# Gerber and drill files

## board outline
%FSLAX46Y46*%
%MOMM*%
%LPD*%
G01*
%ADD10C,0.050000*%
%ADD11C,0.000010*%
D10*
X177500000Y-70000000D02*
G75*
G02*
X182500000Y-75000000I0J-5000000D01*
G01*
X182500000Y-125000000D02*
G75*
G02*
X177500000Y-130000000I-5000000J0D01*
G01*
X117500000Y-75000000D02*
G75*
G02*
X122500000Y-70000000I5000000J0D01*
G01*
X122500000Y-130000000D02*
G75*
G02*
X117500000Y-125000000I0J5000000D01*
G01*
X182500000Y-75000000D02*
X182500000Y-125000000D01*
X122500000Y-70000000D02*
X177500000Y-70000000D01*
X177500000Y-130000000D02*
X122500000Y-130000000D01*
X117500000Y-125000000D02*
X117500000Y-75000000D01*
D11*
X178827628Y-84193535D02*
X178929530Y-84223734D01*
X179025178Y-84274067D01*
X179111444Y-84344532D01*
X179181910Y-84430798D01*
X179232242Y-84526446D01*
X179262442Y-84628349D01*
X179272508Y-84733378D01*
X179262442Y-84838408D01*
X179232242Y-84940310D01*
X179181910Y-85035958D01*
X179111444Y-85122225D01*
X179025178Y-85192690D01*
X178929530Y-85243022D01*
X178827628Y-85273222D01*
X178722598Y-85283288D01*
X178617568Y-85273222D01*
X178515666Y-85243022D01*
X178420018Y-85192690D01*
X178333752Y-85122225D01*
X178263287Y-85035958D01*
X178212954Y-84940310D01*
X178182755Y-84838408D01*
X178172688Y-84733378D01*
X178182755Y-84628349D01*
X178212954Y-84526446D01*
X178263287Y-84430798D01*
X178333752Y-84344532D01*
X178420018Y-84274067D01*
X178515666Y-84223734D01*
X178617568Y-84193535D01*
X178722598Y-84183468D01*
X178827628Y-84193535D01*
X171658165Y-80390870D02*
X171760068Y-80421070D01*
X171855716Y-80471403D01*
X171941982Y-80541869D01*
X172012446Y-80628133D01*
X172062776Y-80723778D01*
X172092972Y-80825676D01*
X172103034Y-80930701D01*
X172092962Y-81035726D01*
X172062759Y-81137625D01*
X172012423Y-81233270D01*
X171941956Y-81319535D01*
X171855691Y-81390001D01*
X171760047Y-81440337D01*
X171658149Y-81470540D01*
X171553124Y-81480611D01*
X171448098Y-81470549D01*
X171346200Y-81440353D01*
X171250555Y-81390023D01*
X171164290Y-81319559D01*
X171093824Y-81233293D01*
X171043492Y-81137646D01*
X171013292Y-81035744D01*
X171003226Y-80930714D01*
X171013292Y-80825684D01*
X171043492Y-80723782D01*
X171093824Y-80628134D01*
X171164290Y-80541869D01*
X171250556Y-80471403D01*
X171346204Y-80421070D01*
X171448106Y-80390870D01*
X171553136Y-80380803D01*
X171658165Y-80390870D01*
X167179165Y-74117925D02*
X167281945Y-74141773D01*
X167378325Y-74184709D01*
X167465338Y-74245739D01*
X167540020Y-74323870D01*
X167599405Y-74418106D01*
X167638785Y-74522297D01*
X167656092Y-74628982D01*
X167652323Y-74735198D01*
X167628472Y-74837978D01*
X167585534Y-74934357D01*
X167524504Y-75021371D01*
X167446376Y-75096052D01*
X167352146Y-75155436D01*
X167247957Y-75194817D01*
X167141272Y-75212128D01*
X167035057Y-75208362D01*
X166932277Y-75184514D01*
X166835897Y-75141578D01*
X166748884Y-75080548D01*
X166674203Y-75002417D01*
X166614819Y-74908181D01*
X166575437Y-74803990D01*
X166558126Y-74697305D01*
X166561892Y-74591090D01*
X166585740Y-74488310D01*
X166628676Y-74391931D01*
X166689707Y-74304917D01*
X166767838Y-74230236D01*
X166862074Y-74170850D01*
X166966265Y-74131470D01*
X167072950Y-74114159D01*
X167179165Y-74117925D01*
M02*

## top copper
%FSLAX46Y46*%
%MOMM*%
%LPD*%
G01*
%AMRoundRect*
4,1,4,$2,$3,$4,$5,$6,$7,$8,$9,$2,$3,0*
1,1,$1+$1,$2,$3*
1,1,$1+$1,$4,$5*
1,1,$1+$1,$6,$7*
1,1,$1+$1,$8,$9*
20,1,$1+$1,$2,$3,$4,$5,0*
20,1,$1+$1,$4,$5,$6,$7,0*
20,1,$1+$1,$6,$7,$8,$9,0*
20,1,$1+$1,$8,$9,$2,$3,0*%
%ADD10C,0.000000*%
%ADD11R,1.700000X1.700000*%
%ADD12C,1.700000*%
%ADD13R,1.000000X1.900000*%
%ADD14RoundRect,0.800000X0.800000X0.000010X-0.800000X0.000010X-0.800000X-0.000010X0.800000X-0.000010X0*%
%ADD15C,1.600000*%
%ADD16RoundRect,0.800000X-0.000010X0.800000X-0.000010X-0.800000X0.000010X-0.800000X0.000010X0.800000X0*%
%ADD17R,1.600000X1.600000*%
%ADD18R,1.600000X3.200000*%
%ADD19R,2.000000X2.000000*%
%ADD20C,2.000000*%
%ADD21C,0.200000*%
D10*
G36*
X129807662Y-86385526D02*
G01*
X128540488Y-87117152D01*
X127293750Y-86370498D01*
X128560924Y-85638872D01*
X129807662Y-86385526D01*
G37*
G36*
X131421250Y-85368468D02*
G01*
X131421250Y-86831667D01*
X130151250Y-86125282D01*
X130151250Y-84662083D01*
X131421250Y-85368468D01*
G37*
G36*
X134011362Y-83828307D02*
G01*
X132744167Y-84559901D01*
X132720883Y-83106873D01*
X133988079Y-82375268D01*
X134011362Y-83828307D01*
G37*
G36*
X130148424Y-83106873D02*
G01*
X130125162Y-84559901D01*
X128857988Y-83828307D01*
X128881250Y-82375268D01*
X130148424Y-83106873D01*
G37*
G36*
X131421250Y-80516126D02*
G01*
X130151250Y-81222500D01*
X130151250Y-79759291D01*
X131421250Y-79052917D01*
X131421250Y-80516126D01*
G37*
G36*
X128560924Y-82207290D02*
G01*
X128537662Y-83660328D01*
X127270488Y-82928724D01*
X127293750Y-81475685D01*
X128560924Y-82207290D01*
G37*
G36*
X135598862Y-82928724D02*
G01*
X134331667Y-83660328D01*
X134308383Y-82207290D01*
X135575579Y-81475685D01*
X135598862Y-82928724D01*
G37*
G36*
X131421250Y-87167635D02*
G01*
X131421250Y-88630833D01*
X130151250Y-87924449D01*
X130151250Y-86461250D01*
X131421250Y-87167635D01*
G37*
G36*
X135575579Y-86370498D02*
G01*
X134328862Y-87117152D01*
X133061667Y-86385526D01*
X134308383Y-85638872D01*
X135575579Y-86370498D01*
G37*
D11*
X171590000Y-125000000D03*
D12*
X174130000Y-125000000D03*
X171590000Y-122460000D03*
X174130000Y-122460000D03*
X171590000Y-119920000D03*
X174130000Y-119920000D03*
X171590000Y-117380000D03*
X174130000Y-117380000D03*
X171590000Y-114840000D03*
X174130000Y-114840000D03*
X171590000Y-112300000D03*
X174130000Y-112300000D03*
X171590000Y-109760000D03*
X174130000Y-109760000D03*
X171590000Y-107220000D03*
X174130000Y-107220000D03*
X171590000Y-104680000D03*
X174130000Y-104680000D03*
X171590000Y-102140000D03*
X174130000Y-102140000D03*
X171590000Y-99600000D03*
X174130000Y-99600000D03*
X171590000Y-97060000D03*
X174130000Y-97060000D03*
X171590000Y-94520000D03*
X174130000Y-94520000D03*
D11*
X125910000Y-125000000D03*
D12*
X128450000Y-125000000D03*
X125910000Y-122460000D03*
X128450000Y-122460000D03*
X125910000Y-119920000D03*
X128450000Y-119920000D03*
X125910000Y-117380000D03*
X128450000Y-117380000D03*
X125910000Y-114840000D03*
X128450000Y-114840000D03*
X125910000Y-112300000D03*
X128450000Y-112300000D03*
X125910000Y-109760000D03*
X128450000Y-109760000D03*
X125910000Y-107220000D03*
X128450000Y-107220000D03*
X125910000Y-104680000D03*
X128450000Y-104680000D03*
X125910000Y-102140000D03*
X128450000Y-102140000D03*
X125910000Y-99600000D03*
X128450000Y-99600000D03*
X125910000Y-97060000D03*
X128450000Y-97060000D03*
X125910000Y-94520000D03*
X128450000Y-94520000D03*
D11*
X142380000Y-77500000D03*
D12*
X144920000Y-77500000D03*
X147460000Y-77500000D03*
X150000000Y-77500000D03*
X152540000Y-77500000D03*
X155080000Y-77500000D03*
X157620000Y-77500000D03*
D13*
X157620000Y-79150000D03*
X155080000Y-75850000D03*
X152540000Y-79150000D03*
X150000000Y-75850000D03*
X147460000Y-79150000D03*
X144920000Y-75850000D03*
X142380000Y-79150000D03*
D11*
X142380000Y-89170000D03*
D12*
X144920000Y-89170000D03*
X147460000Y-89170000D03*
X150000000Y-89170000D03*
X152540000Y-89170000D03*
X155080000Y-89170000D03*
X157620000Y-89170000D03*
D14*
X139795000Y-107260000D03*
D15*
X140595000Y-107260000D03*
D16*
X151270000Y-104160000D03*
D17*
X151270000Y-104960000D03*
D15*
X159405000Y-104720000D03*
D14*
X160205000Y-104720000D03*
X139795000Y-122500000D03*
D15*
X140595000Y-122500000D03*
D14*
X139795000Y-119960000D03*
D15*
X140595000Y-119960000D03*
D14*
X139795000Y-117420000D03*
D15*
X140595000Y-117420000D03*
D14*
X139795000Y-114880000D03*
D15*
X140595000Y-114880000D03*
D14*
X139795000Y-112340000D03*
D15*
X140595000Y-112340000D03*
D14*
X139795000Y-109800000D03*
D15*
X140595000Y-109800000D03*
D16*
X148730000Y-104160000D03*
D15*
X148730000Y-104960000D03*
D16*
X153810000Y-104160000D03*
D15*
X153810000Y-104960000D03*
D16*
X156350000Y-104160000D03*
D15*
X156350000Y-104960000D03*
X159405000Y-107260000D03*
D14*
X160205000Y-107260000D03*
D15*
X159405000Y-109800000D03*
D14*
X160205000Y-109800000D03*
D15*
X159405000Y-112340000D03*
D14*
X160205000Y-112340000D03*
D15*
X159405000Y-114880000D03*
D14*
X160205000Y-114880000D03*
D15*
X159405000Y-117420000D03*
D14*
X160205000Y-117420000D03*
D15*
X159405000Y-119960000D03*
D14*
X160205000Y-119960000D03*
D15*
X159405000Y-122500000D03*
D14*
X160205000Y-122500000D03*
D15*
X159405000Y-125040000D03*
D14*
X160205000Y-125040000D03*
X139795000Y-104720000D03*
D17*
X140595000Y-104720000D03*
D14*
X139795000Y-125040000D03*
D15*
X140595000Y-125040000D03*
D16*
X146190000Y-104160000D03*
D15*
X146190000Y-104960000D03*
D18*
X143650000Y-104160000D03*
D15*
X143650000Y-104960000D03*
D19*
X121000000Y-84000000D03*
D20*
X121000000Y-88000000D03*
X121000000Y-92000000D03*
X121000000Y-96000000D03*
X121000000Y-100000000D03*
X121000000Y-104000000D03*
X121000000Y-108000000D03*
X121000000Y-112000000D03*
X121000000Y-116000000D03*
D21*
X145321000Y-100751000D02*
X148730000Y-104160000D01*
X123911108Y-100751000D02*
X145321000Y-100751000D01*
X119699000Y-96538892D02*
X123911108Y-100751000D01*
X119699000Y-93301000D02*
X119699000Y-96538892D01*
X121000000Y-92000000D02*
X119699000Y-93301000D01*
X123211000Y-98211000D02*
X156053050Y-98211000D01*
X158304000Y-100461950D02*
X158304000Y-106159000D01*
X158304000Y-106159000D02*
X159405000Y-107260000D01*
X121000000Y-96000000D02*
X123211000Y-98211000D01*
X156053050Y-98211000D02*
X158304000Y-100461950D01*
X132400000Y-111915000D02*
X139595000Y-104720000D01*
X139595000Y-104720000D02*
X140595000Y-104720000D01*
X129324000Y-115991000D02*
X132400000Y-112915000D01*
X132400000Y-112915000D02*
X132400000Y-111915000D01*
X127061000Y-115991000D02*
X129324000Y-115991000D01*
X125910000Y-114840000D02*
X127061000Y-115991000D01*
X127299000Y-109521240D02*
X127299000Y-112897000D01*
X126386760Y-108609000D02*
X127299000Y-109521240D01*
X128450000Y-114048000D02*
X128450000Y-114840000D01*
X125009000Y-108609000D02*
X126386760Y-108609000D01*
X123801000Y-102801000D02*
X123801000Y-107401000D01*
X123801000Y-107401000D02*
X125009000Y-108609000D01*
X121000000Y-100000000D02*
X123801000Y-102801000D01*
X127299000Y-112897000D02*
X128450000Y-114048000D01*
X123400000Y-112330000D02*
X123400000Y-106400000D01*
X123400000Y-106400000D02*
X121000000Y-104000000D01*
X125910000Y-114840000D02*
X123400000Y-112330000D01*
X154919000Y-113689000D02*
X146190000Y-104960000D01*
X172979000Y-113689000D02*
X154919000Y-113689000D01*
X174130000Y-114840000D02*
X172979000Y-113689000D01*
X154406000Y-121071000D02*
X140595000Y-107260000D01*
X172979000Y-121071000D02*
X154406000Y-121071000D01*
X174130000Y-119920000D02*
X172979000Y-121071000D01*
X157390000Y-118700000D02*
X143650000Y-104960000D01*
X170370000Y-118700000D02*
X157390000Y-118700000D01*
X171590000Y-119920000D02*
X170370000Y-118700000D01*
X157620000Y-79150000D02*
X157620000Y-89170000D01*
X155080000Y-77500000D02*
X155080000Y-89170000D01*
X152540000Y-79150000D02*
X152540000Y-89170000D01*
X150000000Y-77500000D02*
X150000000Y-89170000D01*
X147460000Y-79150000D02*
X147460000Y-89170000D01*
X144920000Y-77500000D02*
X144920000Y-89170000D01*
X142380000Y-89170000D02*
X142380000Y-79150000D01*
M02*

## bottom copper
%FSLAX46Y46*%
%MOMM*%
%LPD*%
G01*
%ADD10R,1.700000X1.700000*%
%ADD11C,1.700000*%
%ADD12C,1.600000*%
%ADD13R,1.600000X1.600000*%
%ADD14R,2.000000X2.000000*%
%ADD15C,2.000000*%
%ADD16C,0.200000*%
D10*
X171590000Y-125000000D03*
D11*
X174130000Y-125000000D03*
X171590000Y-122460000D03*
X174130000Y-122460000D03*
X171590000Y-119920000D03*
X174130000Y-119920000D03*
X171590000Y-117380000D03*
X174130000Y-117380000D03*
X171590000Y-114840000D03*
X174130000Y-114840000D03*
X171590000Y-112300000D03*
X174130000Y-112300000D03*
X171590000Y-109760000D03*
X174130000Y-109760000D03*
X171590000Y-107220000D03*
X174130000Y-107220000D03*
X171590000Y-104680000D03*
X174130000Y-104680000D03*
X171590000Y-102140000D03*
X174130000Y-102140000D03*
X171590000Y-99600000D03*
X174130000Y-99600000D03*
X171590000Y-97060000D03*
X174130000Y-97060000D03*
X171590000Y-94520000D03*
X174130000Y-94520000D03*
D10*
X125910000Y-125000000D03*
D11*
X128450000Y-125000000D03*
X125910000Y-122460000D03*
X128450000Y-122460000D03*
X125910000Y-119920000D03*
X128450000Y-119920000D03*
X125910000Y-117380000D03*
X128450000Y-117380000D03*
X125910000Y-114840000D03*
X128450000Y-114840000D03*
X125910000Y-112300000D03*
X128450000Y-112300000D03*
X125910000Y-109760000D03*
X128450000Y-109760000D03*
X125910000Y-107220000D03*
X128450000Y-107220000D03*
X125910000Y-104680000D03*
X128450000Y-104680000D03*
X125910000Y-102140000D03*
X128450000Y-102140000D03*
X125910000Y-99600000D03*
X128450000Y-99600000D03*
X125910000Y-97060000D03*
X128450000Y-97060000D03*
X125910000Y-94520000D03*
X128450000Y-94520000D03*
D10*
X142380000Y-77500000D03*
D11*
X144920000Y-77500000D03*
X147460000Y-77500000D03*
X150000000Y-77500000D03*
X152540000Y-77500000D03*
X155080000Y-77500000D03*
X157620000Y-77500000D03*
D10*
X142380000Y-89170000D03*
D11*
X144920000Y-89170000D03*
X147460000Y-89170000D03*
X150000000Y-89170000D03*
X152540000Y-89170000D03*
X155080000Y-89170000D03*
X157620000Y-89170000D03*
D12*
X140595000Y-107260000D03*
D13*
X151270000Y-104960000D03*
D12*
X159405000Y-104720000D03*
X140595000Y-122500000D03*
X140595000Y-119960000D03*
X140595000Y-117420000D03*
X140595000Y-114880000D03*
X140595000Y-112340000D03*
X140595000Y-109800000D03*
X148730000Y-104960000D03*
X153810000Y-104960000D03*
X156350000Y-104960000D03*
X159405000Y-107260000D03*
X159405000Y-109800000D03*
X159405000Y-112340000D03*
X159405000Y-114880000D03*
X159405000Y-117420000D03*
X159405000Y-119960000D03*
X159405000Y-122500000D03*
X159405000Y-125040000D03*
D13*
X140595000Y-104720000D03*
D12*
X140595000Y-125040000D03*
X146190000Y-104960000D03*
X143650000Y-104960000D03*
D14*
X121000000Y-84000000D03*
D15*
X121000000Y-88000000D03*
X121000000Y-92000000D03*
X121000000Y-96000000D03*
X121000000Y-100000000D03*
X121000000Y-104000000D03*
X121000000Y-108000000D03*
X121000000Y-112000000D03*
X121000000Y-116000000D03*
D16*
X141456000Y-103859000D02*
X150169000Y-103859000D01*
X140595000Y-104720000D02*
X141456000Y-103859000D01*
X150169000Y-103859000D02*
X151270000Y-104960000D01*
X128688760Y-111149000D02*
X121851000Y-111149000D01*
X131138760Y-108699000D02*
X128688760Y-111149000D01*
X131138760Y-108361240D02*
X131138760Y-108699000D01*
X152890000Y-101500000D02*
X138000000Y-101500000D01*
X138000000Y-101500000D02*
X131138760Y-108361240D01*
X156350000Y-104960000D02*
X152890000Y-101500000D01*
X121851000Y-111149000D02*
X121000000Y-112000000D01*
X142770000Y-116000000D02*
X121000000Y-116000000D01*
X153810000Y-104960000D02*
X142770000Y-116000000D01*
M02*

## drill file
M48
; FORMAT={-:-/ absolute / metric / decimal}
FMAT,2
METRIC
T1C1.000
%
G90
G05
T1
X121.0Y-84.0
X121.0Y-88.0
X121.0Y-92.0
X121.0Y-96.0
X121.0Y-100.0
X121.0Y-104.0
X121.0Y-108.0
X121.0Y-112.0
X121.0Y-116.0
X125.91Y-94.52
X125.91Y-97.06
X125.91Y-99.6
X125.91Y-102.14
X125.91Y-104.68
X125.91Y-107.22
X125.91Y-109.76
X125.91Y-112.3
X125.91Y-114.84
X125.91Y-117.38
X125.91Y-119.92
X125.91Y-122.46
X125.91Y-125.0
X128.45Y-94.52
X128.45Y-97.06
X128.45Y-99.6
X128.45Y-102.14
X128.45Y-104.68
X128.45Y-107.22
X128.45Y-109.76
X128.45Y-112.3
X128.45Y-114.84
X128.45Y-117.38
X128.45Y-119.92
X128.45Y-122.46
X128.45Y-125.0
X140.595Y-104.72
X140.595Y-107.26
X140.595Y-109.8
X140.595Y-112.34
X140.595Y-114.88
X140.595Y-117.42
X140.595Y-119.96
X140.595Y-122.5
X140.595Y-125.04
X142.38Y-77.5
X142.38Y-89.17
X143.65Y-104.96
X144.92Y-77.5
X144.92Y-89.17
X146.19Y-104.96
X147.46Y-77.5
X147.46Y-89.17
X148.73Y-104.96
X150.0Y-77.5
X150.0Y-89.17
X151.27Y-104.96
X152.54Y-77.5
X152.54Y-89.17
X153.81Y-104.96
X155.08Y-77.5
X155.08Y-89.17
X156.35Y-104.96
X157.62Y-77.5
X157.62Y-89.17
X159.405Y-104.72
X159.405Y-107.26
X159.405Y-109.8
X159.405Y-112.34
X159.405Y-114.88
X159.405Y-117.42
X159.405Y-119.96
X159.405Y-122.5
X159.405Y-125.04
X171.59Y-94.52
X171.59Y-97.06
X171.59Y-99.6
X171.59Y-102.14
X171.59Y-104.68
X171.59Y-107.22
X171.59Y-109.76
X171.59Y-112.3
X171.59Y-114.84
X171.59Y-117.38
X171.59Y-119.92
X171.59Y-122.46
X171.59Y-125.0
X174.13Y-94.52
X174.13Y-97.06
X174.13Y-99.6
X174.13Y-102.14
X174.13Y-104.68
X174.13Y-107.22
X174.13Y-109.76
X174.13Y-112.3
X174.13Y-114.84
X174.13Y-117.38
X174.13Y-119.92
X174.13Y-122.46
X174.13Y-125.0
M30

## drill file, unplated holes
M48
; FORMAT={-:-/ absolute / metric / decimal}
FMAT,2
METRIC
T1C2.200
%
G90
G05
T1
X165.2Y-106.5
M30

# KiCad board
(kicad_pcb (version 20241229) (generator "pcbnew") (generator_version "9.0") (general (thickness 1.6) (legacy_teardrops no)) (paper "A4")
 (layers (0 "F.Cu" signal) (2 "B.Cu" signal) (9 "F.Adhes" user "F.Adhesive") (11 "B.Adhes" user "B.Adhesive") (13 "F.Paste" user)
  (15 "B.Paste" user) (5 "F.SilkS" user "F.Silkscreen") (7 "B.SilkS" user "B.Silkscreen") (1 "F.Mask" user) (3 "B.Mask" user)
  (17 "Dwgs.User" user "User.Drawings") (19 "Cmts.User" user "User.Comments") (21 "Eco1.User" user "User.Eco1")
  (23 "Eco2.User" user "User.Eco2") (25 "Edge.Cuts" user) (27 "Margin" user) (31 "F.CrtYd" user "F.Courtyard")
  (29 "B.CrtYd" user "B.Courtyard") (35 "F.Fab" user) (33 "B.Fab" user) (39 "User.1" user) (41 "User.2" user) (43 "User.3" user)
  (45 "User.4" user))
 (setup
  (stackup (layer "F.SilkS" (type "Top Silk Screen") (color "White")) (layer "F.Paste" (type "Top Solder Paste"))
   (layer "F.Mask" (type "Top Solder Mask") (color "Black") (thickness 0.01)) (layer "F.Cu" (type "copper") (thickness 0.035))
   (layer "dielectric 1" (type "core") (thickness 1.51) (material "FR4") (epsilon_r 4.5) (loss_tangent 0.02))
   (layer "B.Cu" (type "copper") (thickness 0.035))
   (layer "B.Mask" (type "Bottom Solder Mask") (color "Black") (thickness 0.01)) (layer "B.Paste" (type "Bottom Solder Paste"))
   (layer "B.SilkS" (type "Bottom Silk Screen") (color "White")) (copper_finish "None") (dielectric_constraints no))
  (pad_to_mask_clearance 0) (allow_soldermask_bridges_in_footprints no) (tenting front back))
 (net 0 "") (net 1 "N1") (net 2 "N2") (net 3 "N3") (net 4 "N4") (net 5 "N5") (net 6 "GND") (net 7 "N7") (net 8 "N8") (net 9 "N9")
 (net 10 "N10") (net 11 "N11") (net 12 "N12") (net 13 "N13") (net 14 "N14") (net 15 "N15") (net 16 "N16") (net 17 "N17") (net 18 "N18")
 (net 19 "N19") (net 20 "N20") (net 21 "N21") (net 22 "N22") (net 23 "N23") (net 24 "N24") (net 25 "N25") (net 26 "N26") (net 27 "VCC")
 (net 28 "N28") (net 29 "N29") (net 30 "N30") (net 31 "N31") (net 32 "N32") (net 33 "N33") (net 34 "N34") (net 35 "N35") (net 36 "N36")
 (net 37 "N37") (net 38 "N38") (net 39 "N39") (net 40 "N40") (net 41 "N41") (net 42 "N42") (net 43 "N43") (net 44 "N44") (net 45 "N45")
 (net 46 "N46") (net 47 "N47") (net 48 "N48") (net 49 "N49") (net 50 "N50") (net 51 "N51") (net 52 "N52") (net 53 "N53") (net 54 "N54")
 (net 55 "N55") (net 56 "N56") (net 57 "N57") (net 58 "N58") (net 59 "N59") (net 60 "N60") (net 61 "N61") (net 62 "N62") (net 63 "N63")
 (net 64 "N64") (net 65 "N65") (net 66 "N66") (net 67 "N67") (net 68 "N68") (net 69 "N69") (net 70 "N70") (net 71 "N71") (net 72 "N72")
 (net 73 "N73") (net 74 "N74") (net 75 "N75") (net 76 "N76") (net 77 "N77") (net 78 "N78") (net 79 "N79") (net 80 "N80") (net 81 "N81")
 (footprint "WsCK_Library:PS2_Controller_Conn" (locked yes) (layer "F.Cu") (at 121 100)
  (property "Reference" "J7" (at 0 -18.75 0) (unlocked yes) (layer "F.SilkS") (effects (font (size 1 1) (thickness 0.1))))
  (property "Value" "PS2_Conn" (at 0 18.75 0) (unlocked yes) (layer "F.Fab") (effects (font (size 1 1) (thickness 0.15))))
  (pad "1" thru_hole rect (at 0 -16 270) (size 2 2) (drill 1) (layers "*.Cu" "*.Mask") (remove_unused_layers no) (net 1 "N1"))
  (pad "2" thru_hole circle (at 0 -12 270) (size 2 2) (drill 1) (layers "*.Cu" "*.Mask") (remove_unused_layers no) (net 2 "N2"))
  (pad "3" thru_hole circle (at 0 -8 270) (size 2 2) (drill 1) (layers "*.Cu" "*.Mask") (remove_unused_layers no) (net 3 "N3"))
  (pad "4" thru_hole circle (at 0 -4 270) (size 2 2) (drill 1) (layers "*.Cu" "*.Mask") (remove_unused_layers no) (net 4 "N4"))
  (pad "5" thru_hole circle (at 0 0 270) (size 2 2) (drill 1) (layers "*.Cu" "*.Mask") (remove_unused_layers no) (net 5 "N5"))
  (pad "6" thru_hole circle (at 0 4 270) (size 2 2) (drill 1) (layers "*.Cu" "*.Mask") (remove_unused_layers no) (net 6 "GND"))
  (pad "7" thru_hole circle (at 0 8 270) (size 2 2) (drill 1) (layers "*.Cu" "*.Mask") (remove_unused_layers no) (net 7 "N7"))
  (pad "8" thru_hole circle (at 0 12 270) (size 2 2) (drill 1) (layers "*.Cu" "*.Mask") (remove_unused_layers no) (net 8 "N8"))
  (pad "9" thru_hole circle (at 0 16 270) (size 2 2) (drill 1) (layers "*.Cu" "*.Mask") (remove_unused_layers no) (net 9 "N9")))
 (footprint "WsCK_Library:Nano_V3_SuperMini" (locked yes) (layer "F.Cu") (at 150 116.66 180)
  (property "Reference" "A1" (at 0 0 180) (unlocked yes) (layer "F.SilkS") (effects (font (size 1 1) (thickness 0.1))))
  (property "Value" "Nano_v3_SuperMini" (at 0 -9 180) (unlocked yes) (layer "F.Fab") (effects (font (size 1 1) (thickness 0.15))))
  (pad "1" thru_hole circle (at 6.35 11.7 180) (size 1.6 1.6) (drill 1) (layers "*.Cu" "*.Mask") (remove_unused_layers no) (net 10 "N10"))
  (pad "1" smd rect (at 6.35 12.5 270) (size 3.2 1.6) (layers "F.Cu" "F.Mask") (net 10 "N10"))
  (pad "2" thru_hole circle (at 3.81 11.7 180) (size 1.6 1.6) (drill 1) (layers "*.Cu" "*.Mask") (remove_unused_layers no) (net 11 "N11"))
  (pad "2" smd roundrect (at 3.81 12.5 270) (size 3.2 1.6) (layers "F.Cu" "F.Mask") (roundrect_rratio 0.5) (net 11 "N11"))
  (pad "3" thru_hole circle (at 9.405 -8.38 180) (size 1.6 1.6) (drill 1) (layers "*.Cu" "*.Mask") (remove_unused_layers no) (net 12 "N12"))
  (pad "3" smd roundrect (at 10.205 -8.38 180) (size 3.2 1.6) (layers "F.Cu" "F.Mask") (roundrect_rratio 0.5) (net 12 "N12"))
  (pad "4" thru_hole rect (at 9.405 11.94 180) (size 1.6 1.6) (drill 1) (layers "*.Cu" "*.Mask") (remove_unused_layers no) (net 6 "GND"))
  (pad "4" smd roundrect (at 10.205 11.94 180) (size 3.2 1.6) (layers "F.Cu" "F.Mask") (roundrect_rratio 0.5) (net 6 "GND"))
  (pad "6" smd roundrect (at -10.205 -8.38 180) (size 3.2 1.6) (layers "F.Cu" "F.Mask") (roundrect_rratio 0.5) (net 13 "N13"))
  (pad "6" thru_hole circle (at -9.405 -8.38 180) (size 1.6 1.6) (drill 1) (layers "*.Cu" "*.Mask") (remove_unused_layers no) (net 13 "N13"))
  (pad "7" smd roundrect (at -10.205 -5.84 180) (size 3.2 1.6) (layers "F.Cu" "F.Mask") (roundrect_rratio 0.5) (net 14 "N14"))
  (pad "7" thru_hole circle (at -9.405 -5.84 180) (size 1.6 1.6) (drill 1) (layers "*.Cu" "*.Mask") (remove_unused_layers no) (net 14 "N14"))
  (pad "8" smd roundrect (at -10.205 -3.3 180) (size 3.2 1.6) (layers "F.Cu" "F.Mask") (roundrect_rratio 0.5) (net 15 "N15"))
  (pad "8" thru_hole circle (at -9.405 -3.3 180) (size 1.6 1.6) (drill 1) (layers "*.Cu" "*.Mask") (remove_unused_layers no) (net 15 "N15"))
  (pad "9" smd roundrect (at -10.205 -0.76 180) (size 3.2 1.6) (layers "F.Cu" "F.Mask") (roundrect_rratio 0.5) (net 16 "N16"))
  (pad "9" thru_hole circle (at -9.405 -0.76 180) (size 1.6 1.6) (drill 1) (layers "*.Cu" "*.Mask") (remove_unused_layers no) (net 16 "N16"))
  (pad "10" smd roundrect (at -10.205 1.78 180) (size 3.2 1.6) (layers "F.Cu" "F.Mask") (roundrect_rratio 0.5) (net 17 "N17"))
  (pad "10" thru_hole circle (at -9.405 1.78 180) (size 1.6 1.6) (drill 1) (layers "*.Cu" "*.Mask") (remove_unused_layers no) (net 17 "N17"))
  (pad "11" smd roundrect (at -10.205 4.32 180) (size 3.2 1.6) (layers "F.Cu" "F.Mask") (roundrect_rratio 0.5) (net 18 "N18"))
  (pad "11" thru_hole circle (at -9.405 4.32 180) (size 1.6 1.6) (drill 1) (layers "*.Cu" "*.Mask") (remove_unused_layers no) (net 18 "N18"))
  (pad "12" smd roundrect (at -10.205 6.86 180) (size 3.2 1.6) (layers "F.Cu" "F.Mask") (roundrect_rratio 0.5) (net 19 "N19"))
  (pad "12" thru_hole circle (at -9.405 6.86 180) (size 1.6 1.6) (drill 1) (layers "*.Cu" "*.Mask") (remove_unused_layers no) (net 19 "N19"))
  (pad "13" smd roundrect (at -10.205 9.4 180) (size 3.2 1.6) (layers "F.Cu" "F.Mask") (roundrect_rratio 0.5) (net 4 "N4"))
  (pad "13" thru_hole circle (at -9.405 9.4 180) (size 1.6 1.6) (drill 1) (layers "*.Cu" "*.Mask") (remove_unused_layers no) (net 4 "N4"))
  (pad "14" thru_hole circle (at -6.35 11.7 180) (size 1.6 1.6) (drill 1) (layers "*.Cu" "*.Mask") (remove_unused_layers no) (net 8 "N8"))
  (pad "14" smd roundrect (at -6.35 12.5 270) (size 3.2 1.6) (layers "F.Cu" "F.Mask") (roundrect_rratio 0.5) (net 8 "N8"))
  (pad "15" thru_hole circle (at -3.81 11.7 180) (size 1.6 1.6) (drill 1) (layers "*.Cu" "*.Mask") (remove_unused_layers no) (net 9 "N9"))
  (pad "15" smd roundrect (at -3.81 12.5 270) (size 3.2 1.6) (layers "F.Cu" "F.Mask") (roundrect_rratio 0.5) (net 9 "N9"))
  (pad "16" thru_hole circle (at 1.27 11.7 180) (size 1.6 1.6) (drill 1) (layers "*.Cu" "*.Mask") (remove_unused_layers no) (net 3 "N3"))
  (pad "16" smd roundrect (at 1.27 12.5 270) (size 3.2 1.6) (layers "F.Cu" "F.Mask") (roundrect_rratio 0.5) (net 3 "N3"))
  (pad "19" thru_hole circle (at 9.405 6.86 180) (size 1.6 1.6) (drill 1) (layers "*.Cu" "*.Mask") (remove_unused_layers no) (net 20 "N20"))
  (pad "19" smd roundrect (at 10.205 6.86 180) (size 3.2 1.6) (layers "F.Cu" "F.Mask") (roundrect_rratio 0.5) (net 20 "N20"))
  (pad "20" thru_hole circle (at 9.405 4.32 180) (size 1.6 1.6) (drill 1) (layers "*.Cu" "*.Mask") (remove_unused_layers no) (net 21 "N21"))
  (pad "20" smd roundrect (at 10.205 4.32 180) (size 3.2 1.6) (layers "F.Cu" "F.Mask") (roundrect_rratio 0.5) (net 21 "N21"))
  (pad "21" thru_hole circle (at 9.405 1.78 180) (size 1.6 1.6) (drill 1) (layers "*.Cu" "*.Mask") (remove_unused_layers no) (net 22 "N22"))
  (pad "21" smd roundrect (at 10.205 1.78 180) (size 3.2 1.6) (layers "F.Cu" "F.Mask") (roundrect_rratio 0.5) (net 22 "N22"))
  (pad "22" thru_hole circle (at 9.405 -0.76 180) (size 1.6 1.6) (drill 1) (layers "*.Cu" "*.Mask") (remove_unused_layers no) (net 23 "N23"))
  (pad "22" smd roundrect (at 10.205 -0.76 180) (size 3.2 1.6) (layers "F.Cu" "F.Mask") (roundrect_rratio 0.5) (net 23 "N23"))
  (pad "23" thru_hole circle (at 9.405 -3.3 180) (size 1.6 1.6) (drill 1) (layers "*.Cu" "*.Mask") (remove_unused_layers no) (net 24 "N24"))
  (pad "23" smd roundrect (at 10.205 -3.3 180) (size 3.2 1.6) (layers "F.Cu" "F.Mask") (roundrect_rratio 0.5) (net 24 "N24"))
  (pad "24" thru_hole circle (at 9.405 -5.84 180) (size 1.6 1.6) (drill 1) (layers "*.Cu" "*.Mask") (remove_unused_layers no) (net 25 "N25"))
  (pad "24" smd roundrect (at 10.205 -5.84 180) (size 3.2 1.6) (layers "F.Cu" "F.Mask") (roundrect_rratio 0.5) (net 25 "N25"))
  (pad "27" smd roundrect (at -10.205 11.94 180) (size 3.2 1.6) (layers "F.Cu" "F.Mask") (roundrect_rratio 0.5) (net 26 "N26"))
  (pad "27" thru_hole circle (at -9.405 11.94 180) (size 1.6 1.6) (drill 1) (layers "*.Cu" "*.Mask") (remove_unused_layers no)
   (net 26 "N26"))
  (pad "29" thru_hole rect (at -1.27 11.7 180) (size 1.6 1.6) (drill 1) (layers "*.Cu" "*.Mask") (remove_unused_layers no) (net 6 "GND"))
  (pad "29" smd roundrect (at -1.27 12.5 270) (size 3.2 1.6) (layers "F.Cu" "F.Mask") (roundrect_rratio 0.5) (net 6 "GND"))
  (pad "30" thru_hole circle (at 9.405 9.4 180) (size 1.6 1.6) (drill 1) (layers "*.Cu" "*.Mask") (remove_unused_layers no) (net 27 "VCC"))
  (pad "30" smd roundrect (at 10.205 9.4 180) (size 3.2 1.6) (layers "F.Cu" "F.Mask") (roundrect_rratio 0.5) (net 27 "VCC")))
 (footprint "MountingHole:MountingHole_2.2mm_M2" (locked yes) (layer "F.Cu") (at 165.2 106.5)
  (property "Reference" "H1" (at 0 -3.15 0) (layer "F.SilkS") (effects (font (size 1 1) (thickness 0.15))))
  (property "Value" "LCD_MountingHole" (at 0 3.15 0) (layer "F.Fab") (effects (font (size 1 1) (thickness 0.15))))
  (pad "" np_thru_hole circle (at 0 0) (size 2.2 2.2) (drill 2.2) (layers "*.Cu" "*.Mask")))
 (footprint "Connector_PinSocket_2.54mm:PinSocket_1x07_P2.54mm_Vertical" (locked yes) (layer "F.Cu") (at 142.38 77.5 90)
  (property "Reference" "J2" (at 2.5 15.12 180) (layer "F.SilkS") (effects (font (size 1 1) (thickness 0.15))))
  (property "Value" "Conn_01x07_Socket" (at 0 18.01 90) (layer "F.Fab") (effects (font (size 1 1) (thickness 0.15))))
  (pad "1" thru_hole rect (at 0 0 90) (size 1.7 1.7) (drill 1) (layers "*.Cu" "*.Mask") (remove_unused_layers no) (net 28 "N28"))
  (pad "2" thru_hole circle (at 0 2.54 90) (size 1.7 1.7) (drill 1) (layers "*.Cu" "*.Mask") (remove_unused_layers no) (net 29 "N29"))
  (pad "3" thru_hole circle (at 0 5.08 90) (size 1.7 1.7) (drill 1) (layers "*.Cu" "*.Mask") (remove_unused_layers no) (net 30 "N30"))
  (pad "4" thru_hole circle (at 0 7.62 90) (size 1.7 1.7) (drill 1) (layers "*.Cu" "*.Mask") (remove_unused_layers no) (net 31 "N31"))
  (pad "5" thru_hole circle (at 0 10.16 90) (size 1.7 1.7) (drill 1) (layers "*.Cu" "*.Mask") (remove_unused_layers no) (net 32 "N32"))
  (pad "6" thru_hole circle (at 0 12.7 90) (size 1.7 1.7) (drill 1) (layers "*.Cu" "*.Mask") (remove_unused_layers no) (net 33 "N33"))
  (pad "7" thru_hole circle (at 0 15.24 90) (size 1.7 1.7) (drill 1) (layers "*.Cu" "*.Mask") (remove_unused_layers no) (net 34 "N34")))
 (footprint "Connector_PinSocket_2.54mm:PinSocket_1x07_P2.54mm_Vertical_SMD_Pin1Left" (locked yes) (layer "F.Cu") (at 150 77.5 90)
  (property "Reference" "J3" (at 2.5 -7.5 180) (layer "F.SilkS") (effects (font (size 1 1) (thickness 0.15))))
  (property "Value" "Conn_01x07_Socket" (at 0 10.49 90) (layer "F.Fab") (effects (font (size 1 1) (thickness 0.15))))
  (pad "1" smd rect (at -1.65 -7.62 90) (size 1.9 1) (layers "F.Cu" "F.Mask" "F.Paste") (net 28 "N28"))
  (pad "2" smd rect (at 1.65 -5.08 90) (size 1.9 1) (layers "F.Cu" "F.Mask" "F.Paste") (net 29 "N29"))
  (pad "3" smd rect (at -1.65 -2.54 90) (size 1.9 1) (layers "F.Cu" "F.Mask" "F.Paste") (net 30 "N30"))
  (pad "4" smd rect (at 1.65 0 90) (size 1.9 1) (layers "F.Cu" "F.Mask" "F.Paste") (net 31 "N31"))
  (pad "5" smd rect (at -1.65 2.54 90) (size 1.9 1) (layers "F.Cu" "F.Mask" "F.Paste") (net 32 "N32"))
  (pad "6" smd rect (at 1.65 5.08 90) (size 1.9 1) (layers "F.Cu" "F.Mask" "F.Paste") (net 33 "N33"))
  (pad "7" smd rect (at -1.65 7.62 90) (size 1.9 1) (layers "F.Cu" "F.Mask" "F.Paste") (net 34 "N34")))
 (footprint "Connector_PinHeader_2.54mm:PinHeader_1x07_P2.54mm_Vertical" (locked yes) (layer "B.Cu") (at 142.38 89.17 -90)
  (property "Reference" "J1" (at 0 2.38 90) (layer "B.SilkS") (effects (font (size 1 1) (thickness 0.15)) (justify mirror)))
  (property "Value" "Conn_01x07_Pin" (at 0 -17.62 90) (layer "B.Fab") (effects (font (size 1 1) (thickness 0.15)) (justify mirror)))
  (pad "1" thru_hole rect (at 0 0 270) (size 1.7 1.7) (drill 1) (layers "*.Cu" "*.Mask") (remove_unused_layers no) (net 28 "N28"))
  (pad "2" thru_hole circle (at 0 -2.54 270) (size 1.7 1.7) (drill 1) (layers "*.Cu" "*.Mask") (remove_unused_layers no) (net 29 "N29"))
  (pad "3" thru_hole circle (at 0 -5.08 270) (size 1.7 1.7) (drill 1) (layers "*.Cu" "*.Mask") (remove_unused_layers no) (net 30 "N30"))
  (pad "4" thru_hole circle (at 0 -7.62 270) (size 1.7 1.7) (drill 1) (layers "*.Cu" "*.Mask") (remove_unused_layers no) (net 31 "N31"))
  (pad "5" thru_hole circle (at 0 -10.16 270) (size 1.7 1.7) (drill 1) (layers "*.Cu" "*.Mask") (remove_unused_layers no) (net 32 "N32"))
  (pad "6" thru_hole circle (at 0 -12.7 270) (size 1.7 1.7) (drill 1) (layers "*.Cu" "*.Mask") (remove_unused_layers no) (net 33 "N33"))
  (pad "7" thru_hole circle (at 0 -15.24 270) (size 1.7 1.7) (drill 1) (layers "*.Cu" "*.Mask") (remove_unused_layers no) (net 34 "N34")))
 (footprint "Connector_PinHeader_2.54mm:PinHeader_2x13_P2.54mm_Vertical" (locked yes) (layer "B.Cu") (at 171.59 125)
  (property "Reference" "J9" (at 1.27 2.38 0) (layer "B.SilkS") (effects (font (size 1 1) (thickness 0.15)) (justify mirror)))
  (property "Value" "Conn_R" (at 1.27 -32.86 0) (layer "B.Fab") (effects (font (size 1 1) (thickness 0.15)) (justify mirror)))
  (pad "1" thru_hole rect (at 0 0) (size 1.7 1.7) (drill 1) (layers "*.Cu" "*.Mask") (remove_unused_layers no) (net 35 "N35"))
  (pad "2" thru_hole circle (at 2.54 0) (size 1.7 1.7) (drill 1) (layers "*.Cu" "*.Mask") (remove_unused_layers no) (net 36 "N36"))
  (pad "3" thru_hole circle (at 0 -2.54) (size 1.7 1.7) (drill 1) (layers "*.Cu" "*.Mask") (remove_unused_layers no) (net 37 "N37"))
  (pad "4" thru_hole circle (at 2.54 -2.54) (size 1.7 1.7) (drill 1) (layers "*.Cu" "*.Mask") (remove_unused_layers no) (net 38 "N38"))
  (pad "5" thru_hole circle (at 0 -5.08) (size 1.7 1.7) (drill 1) (layers "*.Cu" "*.Mask") (remove_unused_layers no) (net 10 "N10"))
  (pad "6" thru_hole circle (at 2.54 -5.08) (size 1.7 1.7) (drill 1) (layers "*.Cu" "*.Mask") (remove_unused_layers no) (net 27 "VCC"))
  (pad "7" thru_hole circle (at 0 -7.62) (size 1.7 1.7) (drill 1) (layers "*.Cu" "*.Mask") (remove_unused_layers no) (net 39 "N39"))
  (pad "8" thru_hole circle (at 2.54 -7.62) (size 1.7 1.7) (drill 1) (layers "*.Cu" "*.Mask") (remove_unused_layers no) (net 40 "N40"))
  (pad "9" thru_hole circle (at 0 -10.16) (size 1.7 1.7) (drill 1) (layers "*.Cu" "*.Mask") (remove_unused_layers no) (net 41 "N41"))
  (pad "10" thru_hole circle (at 2.54 -10.16) (size 1.7 1.7) (drill 1) (layers "*.Cu" "*.Mask") (remove_unused_layers no) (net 11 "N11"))
  (pad "11" thru_hole circle (at 0 -12.7) (size 1.7 1.7) (drill 1) (layers "*.Cu" "*.Mask") (remove_unused_layers no) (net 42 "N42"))
  (pad "12" thru_hole circle (at 2.54 -12.7) (size 1.7 1.7) (drill 1) (layers "*.Cu" "*.Mask") (remove_unused_layers no) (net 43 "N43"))
  (pad "13" thru_hole circle (at 0 -15.24) (size 1.7 1.7) (drill 1) (layers "*.Cu" "*.Mask") (remove_unused_layers no) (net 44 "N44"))
  (pad "14" thru_hole circle (at 2.54 -15.24) (size 1.7 1.7) (drill 1) (layers "*.Cu" "*.Mask") (remove_unused_layers no) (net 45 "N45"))
  (pad "15" thru_hole circle (at 0 -17.78) (size 1.7 1.7) (drill 1) (layers "*.Cu" "*.Mask") (remove_unused_layers no) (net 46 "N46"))
  (pad "16" thru_hole circle (at 2.54 -17.78) (size 1.7 1.7) (drill 1) (layers "*.Cu" "*.Mask") (remove_unused_layers no) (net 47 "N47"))
  (pad "17" thru_hole circle (at 0 -20.32) (size 1.7 1.7) (drill 1) (layers "*.Cu" "*.Mask") (remove_unused_layers no) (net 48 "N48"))
  (pad "18" thru_hole circle (at 2.54 -20.32) (size 1.7 1.7) (drill 1) (layers "*.Cu" "*.Mask") (remove_unused_layers no) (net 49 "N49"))
  (pad "19" thru_hole circle (at 0 -22.86) (size 1.7 1.7) (drill 1) (layers "*.Cu" "*.Mask") (remove_unused_layers no) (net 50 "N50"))
  (pad "20" thru_hole circle (at 2.54 -22.86) (size 1.7 1.7) (drill 1) (layers "*.Cu" "*.Mask") (remove_unused_layers no) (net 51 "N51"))
  (pad "21" thru_hole circle (at 0 -25.4) (size 1.7 1.7) (drill 1) (layers "*.Cu" "*.Mask") (remove_unused_layers no) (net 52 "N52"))
  (pad "22" thru_hole circle (at 2.54 -25.4) (size 1.7 1.7) (drill 1) (layers "*.Cu" "*.Mask") (remove_unused_layers no) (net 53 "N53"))
  (pad "23" thru_hole circle (at 0 -27.94) (size 1.7 1.7) (drill 1) (layers "*.Cu" "*.Mask") (remove_unused_layers no) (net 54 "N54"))
  (pad "24" thru_hole circle (at 2.54 -27.94) (size 1.7 1.7) (drill 1) (layers "*.Cu" "*.Mask") (remove_unused_layers no) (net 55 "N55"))
  (pad "25" thru_hole circle (at 0 -30.48) (size 1.7 1.7) (drill 1) (layers "*.Cu" "*.Mask") (remove_unused_layers no) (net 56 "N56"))
  (pad "26" thru_hole circle (at 2.54 -30.48) (size 1.7 1.7) (drill 1) (layers "*.Cu" "*.Mask") (remove_unused_layers no) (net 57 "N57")))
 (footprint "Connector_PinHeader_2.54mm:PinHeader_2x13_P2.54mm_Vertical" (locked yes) (layer "B.Cu") (at 125.91 125)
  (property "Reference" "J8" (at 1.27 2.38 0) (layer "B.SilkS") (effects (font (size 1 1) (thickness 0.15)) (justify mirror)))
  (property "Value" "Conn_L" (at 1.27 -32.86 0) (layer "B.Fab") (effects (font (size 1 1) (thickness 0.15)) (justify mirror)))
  (pad "1" thru_hole rect (at 0 0) (size 1.7 1.7) (drill 1) (layers "*.Cu" "*.Mask") (remove_unused_layers no) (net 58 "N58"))
  (pad "2" thru_hole circle (at 2.54 0) (size 1.7 1.7) (drill 1) (layers "*.Cu" "*.Mask") (remove_unused_layers no) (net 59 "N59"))
  (pad "3" thru_hole circle (at 0 -2.54) (size 1.7 1.7) (drill 1) (layers "*.Cu" "*.Mask") (remove_unused_layers no) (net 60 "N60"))
  (pad "4" thru_hole circle (at 2.54 -2.54) (size 1.7 1.7) (drill 1) (layers "*.Cu" "*.Mask") (remove_unused_layers no) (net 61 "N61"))
  (pad "5" thru_hole circle (at 0 -5.08) (size 1.7 1.7) (drill 1) (layers "*.Cu" "*.Mask") (remove_unused_layers no) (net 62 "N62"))
  (pad "6" thru_hole circle (at 2.54 -5.08) (size 1.7 1.7) (drill 1) (layers "*.Cu" "*.Mask") (remove_unused_layers no) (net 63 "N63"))
  (pad "7" thru_hole circle (at 0 -7.62) (size 1.7 1.7) (drill 1) (layers "*.Cu" "*.Mask") (remove_unused_layers no) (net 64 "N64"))
  (pad "8" thru_hole circle (at 2.54 -7.62) (size 1.7 1.7) (drill 1) (layers "*.Cu" "*.Mask") (remove_unused_layers no) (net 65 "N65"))
  (pad "9" thru_hole circle (at 0 -10.16) (size 1.7 1.7) (drill 1) (layers "*.Cu" "*.Mask") (remove_unused_layers no) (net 6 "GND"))
  (pad "10" thru_hole circle (at 2.54 -10.16) (size 1.7 1.7) (drill 1) (layers "*.Cu" "*.Mask") (remove_unused_layers no) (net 5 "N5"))
  (pad "11" thru_hole circle (at 0 -12.7) (size 1.7 1.7) (drill 1) (layers "*.Cu" "*.Mask") (remove_unused_layers no) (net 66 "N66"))
  (pad "12" thru_hole circle (at 2.54 -12.7) (size 1.7 1.7) (drill 1) (layers "*.Cu" "*.Mask") (remove_unused_layers no) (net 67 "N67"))
  (pad "13" thru_hole circle (at 0 -15.24) (size 1.7 1.7) (drill 1) (layers "*.Cu" "*.Mask") (remove_unused_layers no) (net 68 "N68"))
  (pad "14" thru_hole circle (at 2.54 -15.24) (size 1.7 1.7) (drill 1) (layers "*.Cu" "*.Mask") (remove_unused_layers no) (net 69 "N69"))
  (pad "15" thru_hole circle (at 0 -17.78) (size 1.7 1.7) (drill 1) (layers "*.Cu" "*.Mask") (remove_unused_layers no) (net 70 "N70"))
  (pad "16" thru_hole circle (at 2.54 -17.78) (size 1.7 1.7) (drill 1) (layers "*.Cu" "*.Mask") (remove_unused_layers no) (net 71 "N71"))
  (pad "17" thru_hole circle (at 0 -20.32) (size 1.7 1.7) (drill 1) (layers "*.Cu" "*.Mask") (remove_unused_layers no) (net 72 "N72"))
  (pad "18" thru_hole circle (at 2.54 -20.32) (size 1.7 1.7) (drill 1) (layers "*.Cu" "*.Mask") (remove_unused_layers no) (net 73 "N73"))
  (pad "19" thru_hole circle (at 0 -22.86) (size 1.7 1.7) (drill 1) (layers "*.Cu" "*.Mask") (remove_unused_layers no) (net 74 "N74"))
  (pad "20" thru_hole circle (at 2.54 -22.86) (size 1.7 1.7) (drill 1) (layers "*.Cu" "*.Mask") (remove_unused_layers no) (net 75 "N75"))
  (pad "21" thru_hole circle (at 0 -25.4) (size 1.7 1.7) (drill 1) (layers "*.Cu" "*.Mask") (remove_unused_layers no) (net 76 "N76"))
  (pad "22" thru_hole circle (at 2.54 -25.4) (size 1.7 1.7) (drill 1) (layers "*.Cu" "*.Mask") (remove_unused_layers no) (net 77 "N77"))
  (pad "23" thru_hole circle (at 0 -27.94) (size 1.7 1.7) (drill 1) (layers "*.Cu" "*.Mask") (remove_unused_layers no) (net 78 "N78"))
  (pad "24" thru_hole circle (at 2.54 -27.94) (size 1.7 1.7) (drill 1) (layers "*.Cu" "*.Mask") (remove_unused_layers no) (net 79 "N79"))
  (pad "25" thru_hole circle (at 0 -30.48) (size 1.7 1.7) (drill 1) (layers "*.Cu" "*.Mask") (remove_unused_layers no) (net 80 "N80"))
  (pad "26" thru_hole circle (at 2.54 -30.48) (size 1.7 1.7) (drill 1) (layers "*.Cu" "*.Mask") (remove_unused_layers no) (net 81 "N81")))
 (gr_arc (start 122.5 130) (mid 118.964466 128.535534) (end 117.5 125) (stroke (width 0.05) (type default)) (layer "Edge.Cuts"))
 (gr_line (start 182.5 75) (end 182.5 125) (stroke (width 0.05) (type default)) (layer "Edge.Cuts"))
 (gr_arc (start 117.5 75) (mid 118.964466 71.464466) (end 122.5 70) (stroke (width 0.05) (type default)) (layer "Edge.Cuts"))
 (gr_line (start 117.5 125) (end 117.5 75) (stroke (width 0.05) (type default)) (layer "Edge.Cuts"))
 (gr_line (start 177.5 130) (end 122.5 130) (stroke (width 0.05) (type default)) (layer "Edge.Cuts"))
 (gr_arc (start 177.5 70) (mid 181.035534 71.464466) (end 182.5 75) (stroke (width 0.05) (type default)) (layer "Edge.Cuts"))
 (gr_line (start 122.5 70) (end 177.5 70) (stroke (width 0.05) (type default)) (layer "Edge.Cuts"))
 (gr_arc (start 182.5 125) (mid 181.035534 128.535534) (end 177.5 130) (stroke (width 0.05) (type default)) (layer "Edge.Cuts"))
 (segment (start 121 92) (end 119.699 93.301) (width 0.2) (layer "F.Cu") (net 3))
 (segment (start 123.911108 100.751) (end 145.321 100.751) (width 0.2) (layer "F.Cu") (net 3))
 (segment (start 119.699 96.538892) (end 123.911108 100.751) (width 0.2) (layer "F.Cu") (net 3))
 (segment (start 119.699 93.301) (end 119.699 96.538892) (width 0.2) (layer "F.Cu") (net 3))
 (segment (start 145.321 100.751) (end 148.73 104.16) (width 0.2) (layer "F.Cu") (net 3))
 (segment (start 171.59 119.92) (end 170.37 118.7) (width 0.2) (layer "F.Cu") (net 10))
 (segment (start 170.37 118.7) (end 157.39 118.7) (width 0.2) (layer "F.Cu") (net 10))
 (segment (start 157.39 118.7) (end 143.65 104.96) (width 0.2) (layer "F.Cu") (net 10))
 (segment (start 153.81 104.96) (end 142.77 116) (width 0.2) (layer "B.Cu") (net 9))
 (segment (start 142.77 116) (end 121 116) (width 0.2) (layer "B.Cu") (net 9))
 (segment (start 131.13876 108.699) (end 128.68876 111.149) (width 0.2) (layer "B.Cu") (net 8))
 (segment (start 128.68876 111.149) (end 121.851 111.149) (width 0.2) (layer "B.Cu") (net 8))
 (segment (start 121.851 111.149) (end 121 112) (width 0.2) (layer "B.Cu") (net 8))
 (segment (start 152.89 101.5) (end 138 101.5) (width 0.2) (layer "B.Cu") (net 8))
 (segment (start 156.35 104.96) (end 152.89 101.5) (width 0.2) (layer "B.Cu") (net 8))
 (segment (start 138 101.5) (end 131.13876 108.36124) (width 0.2) (layer "B.Cu") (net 8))
 (segment (start 131.13876 108.36124) (end 131.13876 108.699) (width 0.2) (layer "B.Cu") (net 8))
 (segment (start 172.979 113.689) (end 154.919 113.689) (width 0.2) (layer "F.Cu") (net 11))
 (segment (start 154.919 113.689) (end 146.19 104.96) (width 0.2) (layer "F.Cu") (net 11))
 (segment (start 174.13 114.84) (end 172.979 113.689) (width 0.2) (layer "F.Cu") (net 11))
 (segment (start 132.4 111.915) (end 139.595 104.72) (width 0.2) (layer "F.Cu") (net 6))
 (segment (start 123.4 106.4) (end 121 104) (width 0.2) (layer "F.Cu") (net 6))
 (segment (start 125.91 114.84) (end 123.4 112.33) (width 0.2) (layer "F.Cu") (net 6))
 (segment (start 127.061 115.991) (end 129.324 115.991) (width 0.2) (layer "F.Cu") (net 6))
 (segment (start 129.324 115.991) (end 132.4 112.915) (width 0.2) (layer "F.Cu") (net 6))
 (segment (start 123.4 112.33) (end 123.4 106.4) (width 0.2) (layer "F.Cu") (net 6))
 (segment (start 132.4 112.915) (end 132.4 111.915) (width 0.2) (layer "F.Cu") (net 6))
 (segment (start 139.595 104.72) (end 140.595 104.72) (width 0.2) (layer "F.Cu") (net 6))
 (segment (start 125.91 114.84) (end 127.061 115.991) (width 0.2) (layer "F.Cu") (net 6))
 (segment (start 140.595 104.72) (end 141.456 103.859) (width 0.2) (layer "B.Cu") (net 6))
 (segment (start 150.169 103.859) (end 151.27 104.96) (width 0.2) (layer "B.Cu") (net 6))
 (segment (start 141.456 103.859) (end 150.169 103.859) (width 0.2) (layer "B.Cu") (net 6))
 (segment (start 158.304 106.159) (end 159.405 107.26) (width 0.2) (layer "F.Cu") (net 4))
 (segment (start 123.211 98.211) (end 156.05305 98.211) (width 0.2) (layer "F.Cu") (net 4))
 (segment (start 156.05305 98.211) (end 158.304 100.46195) (width 0.2) (layer "F.Cu") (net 4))
 (segment (start 158.304 100.46195) (end 158.304 106.159) (width 0.2) (layer "F.Cu") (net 4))
 (segment (start 121 96) (end 123.211 98.211) (width 0.2) (layer "F.Cu") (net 4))
 (segment (start 152.54 79.15) (end 152.54 89.17) (width 0.2) (layer "F.Cu") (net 32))
 (segment (start 157.62 79.15) (end 157.62 89.17) (width 0.2) (layer "F.Cu") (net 34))
 (segment (start 147.46 79.15) (end 147.46 89.17) (width 0.2) (layer "F.Cu") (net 30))
 (segment (start 142.38 89.17) (end 142.38 79.15) (width 0.2) (layer "F.Cu") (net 28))
 (segment (start 144.92 77.5) (end 144.92 89.17) (width 0.2) (layer "F.Cu") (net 29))
 (segment (start 150 77.5) (end 150 89.17) (width 0.2) (layer "F.Cu") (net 31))
 (segment (start 155.08 77.5) (end 155.08 89.17) (width 0.2) (layer "F.Cu") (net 33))
 (segment (start 172.979 121.071) (end 154.406 121.071) (width 0.2) (layer "F.Cu") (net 27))
 (segment (start 174.13 119.92) (end 172.979 121.071) (width 0.2) (layer "F.Cu") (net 27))
 (segment (start 154.406 121.071) (end 140.595 107.26) (width 0.2) (layer "F.Cu") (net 27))
 (segment (start 126.38676 108.609) (end 127.299 109.52124) (width 0.2) (layer "F.Cu") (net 5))
 (segment (start 121 100) (end 123.801 102.801) (width 0.2) (layer "F.Cu") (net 5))
 (segment (start 123.801 102.801) (end 123.801 107.401) (width 0.2) (layer "F.Cu") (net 5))
 (segment (start 127.299 109.52124) (end 127.299 112.897) (width 0.2) (layer "F.Cu") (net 5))
 (segment (start 125.009 108.609) (end 126.38676 108.609) (width 0.2) (layer "F.Cu") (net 5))
 (segment (start 127.299 112.897) (end 128.45 114.048) (width 0.2) (layer "F.Cu") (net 5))
 (segment (start 123.801 107.401) (end 125.009 108.609) (width 0.2) (layer "F.Cu") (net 5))
 (segment (start 128.45 114.048) (end 128.45 114.84) (width 0.2) (layer "F.Cu") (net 5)))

